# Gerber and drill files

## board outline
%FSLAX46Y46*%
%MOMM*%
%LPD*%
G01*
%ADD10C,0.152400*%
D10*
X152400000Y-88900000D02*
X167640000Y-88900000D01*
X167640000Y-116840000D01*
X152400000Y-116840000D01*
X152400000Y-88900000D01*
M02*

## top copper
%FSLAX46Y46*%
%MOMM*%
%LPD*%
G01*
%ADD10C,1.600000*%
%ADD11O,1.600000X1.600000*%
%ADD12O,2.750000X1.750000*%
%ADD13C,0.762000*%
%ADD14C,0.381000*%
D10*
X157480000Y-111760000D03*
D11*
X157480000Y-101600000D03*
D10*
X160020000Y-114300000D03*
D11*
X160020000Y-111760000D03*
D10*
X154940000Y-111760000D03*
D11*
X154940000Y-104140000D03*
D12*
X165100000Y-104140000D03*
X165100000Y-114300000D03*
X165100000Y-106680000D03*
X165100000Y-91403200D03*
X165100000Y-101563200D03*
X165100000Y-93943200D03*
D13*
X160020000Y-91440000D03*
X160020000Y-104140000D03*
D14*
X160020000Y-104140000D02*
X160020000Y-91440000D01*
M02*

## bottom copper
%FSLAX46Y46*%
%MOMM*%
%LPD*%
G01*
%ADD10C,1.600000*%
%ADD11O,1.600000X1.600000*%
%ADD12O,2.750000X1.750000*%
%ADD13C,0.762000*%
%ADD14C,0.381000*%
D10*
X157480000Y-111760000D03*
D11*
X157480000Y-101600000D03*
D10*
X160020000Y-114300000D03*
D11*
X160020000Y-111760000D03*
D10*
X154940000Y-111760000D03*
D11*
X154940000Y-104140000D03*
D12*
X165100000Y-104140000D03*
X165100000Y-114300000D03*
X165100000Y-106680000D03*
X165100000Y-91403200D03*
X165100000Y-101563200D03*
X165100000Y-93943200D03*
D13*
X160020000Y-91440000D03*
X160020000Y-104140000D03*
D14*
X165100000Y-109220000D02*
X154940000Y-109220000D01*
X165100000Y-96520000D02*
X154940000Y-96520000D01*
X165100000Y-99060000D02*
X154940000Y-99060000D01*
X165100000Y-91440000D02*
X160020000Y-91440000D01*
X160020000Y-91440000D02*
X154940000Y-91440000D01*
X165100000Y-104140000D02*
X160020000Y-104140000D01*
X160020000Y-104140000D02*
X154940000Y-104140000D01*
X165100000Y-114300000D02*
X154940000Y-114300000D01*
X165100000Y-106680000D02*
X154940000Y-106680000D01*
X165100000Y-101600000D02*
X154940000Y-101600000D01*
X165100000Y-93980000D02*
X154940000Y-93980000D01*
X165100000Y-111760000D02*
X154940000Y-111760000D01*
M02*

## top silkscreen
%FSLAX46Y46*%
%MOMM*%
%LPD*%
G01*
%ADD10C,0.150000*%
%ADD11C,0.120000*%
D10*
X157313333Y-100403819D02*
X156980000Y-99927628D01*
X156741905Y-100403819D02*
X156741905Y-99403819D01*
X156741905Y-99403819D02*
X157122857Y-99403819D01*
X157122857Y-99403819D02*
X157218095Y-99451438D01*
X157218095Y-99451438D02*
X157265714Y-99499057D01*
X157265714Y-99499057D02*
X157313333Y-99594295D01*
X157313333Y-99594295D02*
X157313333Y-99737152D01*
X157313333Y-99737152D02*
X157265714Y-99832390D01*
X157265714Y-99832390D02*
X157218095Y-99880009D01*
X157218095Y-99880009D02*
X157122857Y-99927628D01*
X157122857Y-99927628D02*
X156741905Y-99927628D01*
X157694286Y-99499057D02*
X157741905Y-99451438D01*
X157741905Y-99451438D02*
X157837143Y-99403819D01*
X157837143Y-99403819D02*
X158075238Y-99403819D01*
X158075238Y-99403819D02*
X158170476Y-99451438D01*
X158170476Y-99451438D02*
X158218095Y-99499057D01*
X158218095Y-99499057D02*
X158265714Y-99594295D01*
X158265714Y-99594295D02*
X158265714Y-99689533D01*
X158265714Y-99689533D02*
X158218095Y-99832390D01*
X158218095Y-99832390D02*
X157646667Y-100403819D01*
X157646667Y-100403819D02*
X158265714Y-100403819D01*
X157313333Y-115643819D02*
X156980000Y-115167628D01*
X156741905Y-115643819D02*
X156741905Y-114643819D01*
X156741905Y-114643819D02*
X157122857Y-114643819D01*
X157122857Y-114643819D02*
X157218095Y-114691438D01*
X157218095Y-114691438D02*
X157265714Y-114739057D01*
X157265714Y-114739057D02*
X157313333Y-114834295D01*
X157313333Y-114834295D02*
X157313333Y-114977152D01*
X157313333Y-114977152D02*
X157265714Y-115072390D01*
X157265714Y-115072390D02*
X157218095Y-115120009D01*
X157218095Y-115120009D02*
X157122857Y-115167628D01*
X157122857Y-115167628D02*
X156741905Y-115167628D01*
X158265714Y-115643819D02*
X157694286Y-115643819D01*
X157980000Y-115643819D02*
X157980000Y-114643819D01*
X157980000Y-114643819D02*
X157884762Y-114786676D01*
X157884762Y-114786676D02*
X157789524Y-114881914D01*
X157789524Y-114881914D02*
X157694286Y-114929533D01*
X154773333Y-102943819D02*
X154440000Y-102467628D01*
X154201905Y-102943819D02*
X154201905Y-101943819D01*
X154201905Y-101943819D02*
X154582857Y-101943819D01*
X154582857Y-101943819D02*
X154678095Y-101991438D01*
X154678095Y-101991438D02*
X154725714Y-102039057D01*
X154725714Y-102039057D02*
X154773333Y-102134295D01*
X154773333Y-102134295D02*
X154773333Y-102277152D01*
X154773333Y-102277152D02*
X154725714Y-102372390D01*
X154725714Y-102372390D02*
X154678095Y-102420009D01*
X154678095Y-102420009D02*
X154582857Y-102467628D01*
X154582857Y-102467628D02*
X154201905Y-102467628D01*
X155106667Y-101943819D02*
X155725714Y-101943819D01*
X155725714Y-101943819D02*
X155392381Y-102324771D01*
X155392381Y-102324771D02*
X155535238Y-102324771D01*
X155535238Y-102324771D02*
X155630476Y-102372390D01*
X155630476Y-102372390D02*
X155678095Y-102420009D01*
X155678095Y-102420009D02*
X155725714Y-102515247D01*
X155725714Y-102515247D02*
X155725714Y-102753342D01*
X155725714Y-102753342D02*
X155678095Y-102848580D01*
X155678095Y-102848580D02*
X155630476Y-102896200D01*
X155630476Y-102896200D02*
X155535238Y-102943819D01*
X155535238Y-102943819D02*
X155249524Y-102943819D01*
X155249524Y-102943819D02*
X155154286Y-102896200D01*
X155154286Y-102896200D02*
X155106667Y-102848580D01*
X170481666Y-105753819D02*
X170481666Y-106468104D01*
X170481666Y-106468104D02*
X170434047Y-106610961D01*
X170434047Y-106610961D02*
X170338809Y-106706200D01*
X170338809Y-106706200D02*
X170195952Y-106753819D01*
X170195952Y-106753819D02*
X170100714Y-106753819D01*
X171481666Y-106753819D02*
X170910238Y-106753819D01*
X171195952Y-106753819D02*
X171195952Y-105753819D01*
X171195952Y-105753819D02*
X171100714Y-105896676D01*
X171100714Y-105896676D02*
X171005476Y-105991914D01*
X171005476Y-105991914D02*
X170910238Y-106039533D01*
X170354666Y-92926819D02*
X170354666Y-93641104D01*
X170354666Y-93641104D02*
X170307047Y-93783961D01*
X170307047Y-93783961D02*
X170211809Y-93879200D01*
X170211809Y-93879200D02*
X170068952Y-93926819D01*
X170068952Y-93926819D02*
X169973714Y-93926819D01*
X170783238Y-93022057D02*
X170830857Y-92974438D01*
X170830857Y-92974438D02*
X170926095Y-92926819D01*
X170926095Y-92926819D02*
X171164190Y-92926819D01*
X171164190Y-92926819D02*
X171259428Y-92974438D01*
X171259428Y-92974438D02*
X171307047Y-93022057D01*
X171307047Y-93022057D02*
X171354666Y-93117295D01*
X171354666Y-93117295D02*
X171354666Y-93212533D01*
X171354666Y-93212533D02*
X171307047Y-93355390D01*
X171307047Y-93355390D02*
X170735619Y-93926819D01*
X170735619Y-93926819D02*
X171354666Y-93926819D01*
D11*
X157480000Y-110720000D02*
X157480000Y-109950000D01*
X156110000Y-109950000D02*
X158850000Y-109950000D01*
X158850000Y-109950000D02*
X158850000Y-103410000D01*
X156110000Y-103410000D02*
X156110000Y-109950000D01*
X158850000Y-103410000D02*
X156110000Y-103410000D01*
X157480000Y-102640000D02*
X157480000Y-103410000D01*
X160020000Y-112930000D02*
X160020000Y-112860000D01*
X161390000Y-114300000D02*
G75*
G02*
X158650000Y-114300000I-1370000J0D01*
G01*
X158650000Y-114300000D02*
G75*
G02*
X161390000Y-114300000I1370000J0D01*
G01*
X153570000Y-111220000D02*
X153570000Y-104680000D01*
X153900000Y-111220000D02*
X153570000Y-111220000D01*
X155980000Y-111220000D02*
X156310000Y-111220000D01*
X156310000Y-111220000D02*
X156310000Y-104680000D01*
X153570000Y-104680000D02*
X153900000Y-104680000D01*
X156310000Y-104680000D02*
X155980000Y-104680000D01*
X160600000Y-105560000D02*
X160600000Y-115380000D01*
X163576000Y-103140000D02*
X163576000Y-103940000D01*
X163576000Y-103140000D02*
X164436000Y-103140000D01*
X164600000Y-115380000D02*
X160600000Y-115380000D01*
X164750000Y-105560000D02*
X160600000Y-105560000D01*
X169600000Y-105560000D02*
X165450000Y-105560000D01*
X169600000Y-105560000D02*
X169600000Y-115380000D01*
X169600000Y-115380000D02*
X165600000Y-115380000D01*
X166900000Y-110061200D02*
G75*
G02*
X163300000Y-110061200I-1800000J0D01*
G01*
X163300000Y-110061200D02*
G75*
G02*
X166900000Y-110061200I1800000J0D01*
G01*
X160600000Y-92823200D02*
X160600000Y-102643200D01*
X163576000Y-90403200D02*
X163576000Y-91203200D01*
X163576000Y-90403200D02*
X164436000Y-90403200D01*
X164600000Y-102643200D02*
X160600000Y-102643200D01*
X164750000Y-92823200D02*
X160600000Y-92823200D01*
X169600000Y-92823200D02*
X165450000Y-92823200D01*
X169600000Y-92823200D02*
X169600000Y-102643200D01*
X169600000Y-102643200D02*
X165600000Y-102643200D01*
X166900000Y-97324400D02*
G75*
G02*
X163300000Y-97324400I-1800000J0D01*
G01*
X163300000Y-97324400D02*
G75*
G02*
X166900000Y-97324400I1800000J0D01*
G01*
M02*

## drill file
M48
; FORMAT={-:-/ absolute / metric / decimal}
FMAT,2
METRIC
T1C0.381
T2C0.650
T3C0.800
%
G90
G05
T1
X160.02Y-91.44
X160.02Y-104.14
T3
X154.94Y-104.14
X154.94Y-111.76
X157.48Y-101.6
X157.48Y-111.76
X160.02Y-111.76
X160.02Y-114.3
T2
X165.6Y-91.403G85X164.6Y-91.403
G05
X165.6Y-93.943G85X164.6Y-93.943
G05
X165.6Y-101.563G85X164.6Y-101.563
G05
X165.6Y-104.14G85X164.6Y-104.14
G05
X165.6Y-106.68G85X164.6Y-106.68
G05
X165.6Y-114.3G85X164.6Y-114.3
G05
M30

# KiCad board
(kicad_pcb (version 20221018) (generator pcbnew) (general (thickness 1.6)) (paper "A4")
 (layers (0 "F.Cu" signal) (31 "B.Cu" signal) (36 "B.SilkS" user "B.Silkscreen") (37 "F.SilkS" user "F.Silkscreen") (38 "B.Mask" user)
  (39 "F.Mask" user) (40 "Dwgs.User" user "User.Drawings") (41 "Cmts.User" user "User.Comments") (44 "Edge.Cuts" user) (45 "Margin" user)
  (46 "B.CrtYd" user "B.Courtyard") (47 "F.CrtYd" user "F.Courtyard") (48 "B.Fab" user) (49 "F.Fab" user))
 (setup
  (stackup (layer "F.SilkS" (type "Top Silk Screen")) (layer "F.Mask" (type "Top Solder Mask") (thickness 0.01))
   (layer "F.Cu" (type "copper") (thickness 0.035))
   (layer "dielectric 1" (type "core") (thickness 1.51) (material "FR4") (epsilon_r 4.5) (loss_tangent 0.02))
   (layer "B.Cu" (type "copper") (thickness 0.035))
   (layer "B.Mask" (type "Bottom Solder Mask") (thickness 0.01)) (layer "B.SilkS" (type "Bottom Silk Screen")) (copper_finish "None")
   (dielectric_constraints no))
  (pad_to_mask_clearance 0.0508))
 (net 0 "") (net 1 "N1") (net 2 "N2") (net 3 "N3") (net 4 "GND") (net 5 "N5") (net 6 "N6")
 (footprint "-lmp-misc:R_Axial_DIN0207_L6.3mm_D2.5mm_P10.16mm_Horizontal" (layer "F.Cu") (at 157.48 111.76 90)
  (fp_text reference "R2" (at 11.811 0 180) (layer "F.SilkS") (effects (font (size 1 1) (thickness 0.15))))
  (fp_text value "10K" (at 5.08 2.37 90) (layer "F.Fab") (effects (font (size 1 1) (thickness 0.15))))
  (fp_line (start 1.04 0) (end 1.81 0) (stroke (width 0.12) (type solid)) (layer "F.SilkS"))
  (fp_line (start 1.81 -1.37) (end 1.81 1.37) (stroke (width 0.12) (type solid)) (layer "F.SilkS"))
  (fp_line (start 1.81 1.37) (end 8.35 1.37) (stroke (width 0.12) (type solid)) (layer "F.SilkS"))
  (fp_line (start 8.35 -1.37) (end 1.81 -1.37) (stroke (width 0.12) (type solid)) (layer "F.SilkS"))
  (fp_line (start 8.35 1.37) (end 8.35 -1.37) (stroke (width 0.12) (type solid)) (layer "F.SilkS"))
  (fp_line (start 9.12 0) (end 8.35 0) (stroke (width 0.12) (type solid)) (layer "F.SilkS"))
  (pad "1" thru_hole circle (at 0 0 90) (size 1.6 1.6) (drill 0.8) (layers "*.Cu" "*.Mask") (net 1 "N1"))
  (pad "2" thru_hole oval (at 10.16 0 90) (size 1.6 1.6) (drill 0.8) (layers "*.Cu" "*.Mask") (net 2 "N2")))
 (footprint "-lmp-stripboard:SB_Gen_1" (layer "F.Cu") (at 160.02 114.3 90)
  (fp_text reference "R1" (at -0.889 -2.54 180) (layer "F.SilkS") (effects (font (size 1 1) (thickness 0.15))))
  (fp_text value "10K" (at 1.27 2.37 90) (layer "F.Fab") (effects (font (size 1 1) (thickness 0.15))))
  (fp_line (start 1.37 0) (end 1.44 0) (stroke (width 0.12) (type solid)) (layer "F.SilkS"))
  (fp_circle (center 0 0) (end 1.37 0) (stroke (width 0.12) (type solid)) (fill none) (layer "F.SilkS"))
  (pad "1" thru_hole circle (at 0 0 90) (size 1.6 1.6) (drill 0.8) (layers "*.Cu" "*.Mask") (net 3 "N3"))
  (pad "2" thru_hole oval (at 2.54 0 90) (size 1.6 1.6) (drill 0.8) (layers "*.Cu" "*.Mask") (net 1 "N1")))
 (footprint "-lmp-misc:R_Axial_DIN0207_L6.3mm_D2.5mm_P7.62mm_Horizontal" (layer "F.Cu") (at 154.94 111.76 90)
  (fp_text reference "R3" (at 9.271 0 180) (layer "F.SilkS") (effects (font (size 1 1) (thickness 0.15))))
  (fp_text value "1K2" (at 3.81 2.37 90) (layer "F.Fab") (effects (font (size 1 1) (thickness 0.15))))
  (fp_line (start 0.54 -1.37) (end 7.08 -1.37) (stroke (width 0.12) (type solid)) (layer "F.SilkS"))
  (fp_line (start 0.54 -1.04) (end 0.54 -1.37) (stroke (width 0.12) (type solid)) (layer "F.SilkS"))
  (fp_line (start 0.54 1.04) (end 0.54 1.37) (stroke (width 0.12) (type solid)) (layer "F.SilkS"))
  (fp_line (start 0.54 1.37) (end 7.08 1.37) (stroke (width 0.12) (type solid)) (layer "F.SilkS"))
  (fp_line (start 7.08 -1.37) (end 7.08 -1.04) (stroke (width 0.12) (type solid)) (layer "F.SilkS"))
  (fp_line (start 7.08 1.37) (end 7.08 1.04) (stroke (width 0.12) (type solid)) (layer "F.SilkS"))
  (pad "1" thru_hole circle (at 0 0 90) (size 1.6 1.6) (drill 0.8) (layers "*.Cu" "*.Mask") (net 1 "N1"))
  (pad "2" thru_hole oval (at 7.62 0 90) (size 1.6 1.6) (drill 0.8) (layers "*.Cu" "*.Mask") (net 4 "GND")))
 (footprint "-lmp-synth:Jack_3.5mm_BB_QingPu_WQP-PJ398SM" (layer "F.Cu") (at 165.1 104.14)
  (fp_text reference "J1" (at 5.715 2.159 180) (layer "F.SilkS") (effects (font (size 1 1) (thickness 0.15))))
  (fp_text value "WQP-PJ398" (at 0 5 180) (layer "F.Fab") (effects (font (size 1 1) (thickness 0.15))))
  (fp_line (start -4.5 1.42) (end -4.5 11.24) (stroke (width 0.12) (type solid)) (layer "F.SilkS"))
  (fp_line (start -1.524 -1) (end -1.524 -0.2) (stroke (width 0.12) (type solid)) (layer "F.SilkS"))
  (fp_line (start -1.524 -1) (end -0.664 -1) (stroke (width 0.12) (type solid)) (layer "F.SilkS"))
  (fp_line (start -0.5 11.24) (end -4.5 11.24) (stroke (width 0.12) (type solid)) (layer "F.SilkS"))
  (fp_line (start -0.35 1.42) (end -4.5 1.42) (stroke (width 0.12) (type solid)) (layer "F.SilkS"))
  (fp_line (start 4.5 1.42) (end 0.35 1.42) (stroke (width 0.12) (type solid)) (layer "F.SilkS"))
  (fp_line (start 4.5 1.42) (end 4.5 11.24) (stroke (width 0.12) (type solid)) (layer "F.SilkS"))
  (fp_line (start 4.5 11.24) (end 0.5 11.24) (stroke (width 0.12) (type solid)) (layer "F.SilkS"))
  (fp_circle (center 0 5.9212) (end 1.8 5.9212) (stroke (width 0.12) (type solid)) (fill none) (layer "F.SilkS"))
  (pad "S" thru_hole oval (at 0 0 180) (size 2.75 1.75) (drill oval 1.65 0.65) (layers "*.Cu" "*.Mask") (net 4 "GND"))
  (pad "T" thru_hole oval (at 0 10.16 180) (size 2.75 1.75) (drill oval 1.65 0.65) (layers "*.Cu" "*.Mask") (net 3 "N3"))
  (pad "TN" thru_hole oval (at 0 2.54 180) (size 2.75 1.75) (drill oval 1.65 0.65) (layers "*.Cu" "*.Mask") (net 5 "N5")))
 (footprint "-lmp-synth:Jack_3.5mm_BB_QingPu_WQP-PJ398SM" (layer "F.Cu") (at 165.1 91.4032)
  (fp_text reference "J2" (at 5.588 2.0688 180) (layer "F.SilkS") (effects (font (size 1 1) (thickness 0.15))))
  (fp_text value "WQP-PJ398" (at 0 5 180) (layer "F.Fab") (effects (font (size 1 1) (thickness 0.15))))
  (fp_line (start -4.5 1.42) (end -4.5 11.24) (stroke (width 0.12) (type solid)) (layer "F.SilkS"))
  (fp_line (start -1.524 -1) (end -1.524 -0.2) (stroke (width 0.12) (type solid)) (layer "F.SilkS"))
  (fp_line (start -1.524 -1) (end -0.664 -1) (stroke (width 0.12) (type solid)) (layer "F.SilkS"))
  (fp_line (start -0.5 11.24) (end -4.5 11.24) (stroke (width 0.12) (type solid)) (layer "F.SilkS"))
  (fp_line (start -0.35 1.42) (end -4.5 1.42) (stroke (width 0.12) (type solid)) (layer "F.SilkS"))
  (fp_line (start 4.5 1.42) (end 0.35 1.42) (stroke (width 0.12) (type solid)) (layer "F.SilkS"))
  (fp_line (start 4.5 1.42) (end 4.5 11.24) (stroke (width 0.12) (type solid)) (layer "F.SilkS"))
  (fp_line (start 4.5 11.24) (end 0.5 11.24) (stroke (width 0.12) (type solid)) (layer "F.SilkS"))
  (fp_circle (center 0 5.9212) (end 1.8 5.9212) (stroke (width 0.12) (type solid)) (fill none) (layer "F.SilkS"))
  (pad "S" thru_hole oval (at 0 0 180) (size 2.75 1.75) (drill oval 1.65 0.65) (layers "*.Cu" "*.Mask") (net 4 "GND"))
  (pad "T" thru_hole oval (at 0 10.16 180) (size 2.75 1.75) (drill oval 1.65 0.65) (layers "*.Cu" "*.Mask") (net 2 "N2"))
  (pad "TN" thru_hole oval (at 0 2.54 180) (size 2.75 1.75) (drill oval 1.65 0.65) (layers "*.Cu" "*.Mask") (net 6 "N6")))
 (gr_rect (start 152.4 88.9) (end 167.64 116.84) (stroke (width 0.1524) (type default)) (fill none) (layer "Edge.Cuts"))
 (segment (start 165.1 109.22) (end 154.94 109.22) (width 0.381) (layer "B.Cu") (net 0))
 (segment (start 165.1 96.52) (end 154.94 96.52) (width 0.381) (layer "B.Cu") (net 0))
 (segment (start 165.1 99.06) (end 154.94 99.06) (width 0.381) (layer "B.Cu") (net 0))
 (segment (start 160.02 104.14) (end 160.02 91.44) (width 0.381) (layer "F.Cu") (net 4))
 (via (at 160.02 91.44) (size 0.762) (drill 0.381) (layers "F.Cu" "B.Cu") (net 4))
 (via (at 160.02 104.14) (size 0.762) (drill 0.381) (layers "F.Cu" "B.Cu") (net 4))
 (segment (start 165.1 91.44) (end 160.02 91.44) (width 0.381) (layer "B.Cu") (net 4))
 (segment (start 160.02 91.44) (end 154.94 91.44) (width 0.381) (layer "B.Cu") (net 4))
 (segment (start 165.1 104.14) (end 160.02 104.14) (width 0.381) (layer "B.Cu") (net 4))
 (segment (start 160.02 104.14) (end 154.94 104.14) (width 0.381) (layer "B.Cu") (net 4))
 (segment (start 165.1 114.3) (end 154.94 114.3) (width 0.381) (layer "B.Cu") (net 3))
 (segment (start 165.1 106.68) (end 154.94 106.68) (width 0.381) (layer "B.Cu") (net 5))
 (segment (start 165.1 101.6) (end 154.94 101.6) (width 0.381) (layer "B.Cu") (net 2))
 (segment (start 165.1 93.98) (end 154.94 93.98) (width 0.381) (layer "B.Cu") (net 6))
 (segment (start 165.1 111.76) (end 154.94 111.76) (width 0.381) (layer "B.Cu") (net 1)))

